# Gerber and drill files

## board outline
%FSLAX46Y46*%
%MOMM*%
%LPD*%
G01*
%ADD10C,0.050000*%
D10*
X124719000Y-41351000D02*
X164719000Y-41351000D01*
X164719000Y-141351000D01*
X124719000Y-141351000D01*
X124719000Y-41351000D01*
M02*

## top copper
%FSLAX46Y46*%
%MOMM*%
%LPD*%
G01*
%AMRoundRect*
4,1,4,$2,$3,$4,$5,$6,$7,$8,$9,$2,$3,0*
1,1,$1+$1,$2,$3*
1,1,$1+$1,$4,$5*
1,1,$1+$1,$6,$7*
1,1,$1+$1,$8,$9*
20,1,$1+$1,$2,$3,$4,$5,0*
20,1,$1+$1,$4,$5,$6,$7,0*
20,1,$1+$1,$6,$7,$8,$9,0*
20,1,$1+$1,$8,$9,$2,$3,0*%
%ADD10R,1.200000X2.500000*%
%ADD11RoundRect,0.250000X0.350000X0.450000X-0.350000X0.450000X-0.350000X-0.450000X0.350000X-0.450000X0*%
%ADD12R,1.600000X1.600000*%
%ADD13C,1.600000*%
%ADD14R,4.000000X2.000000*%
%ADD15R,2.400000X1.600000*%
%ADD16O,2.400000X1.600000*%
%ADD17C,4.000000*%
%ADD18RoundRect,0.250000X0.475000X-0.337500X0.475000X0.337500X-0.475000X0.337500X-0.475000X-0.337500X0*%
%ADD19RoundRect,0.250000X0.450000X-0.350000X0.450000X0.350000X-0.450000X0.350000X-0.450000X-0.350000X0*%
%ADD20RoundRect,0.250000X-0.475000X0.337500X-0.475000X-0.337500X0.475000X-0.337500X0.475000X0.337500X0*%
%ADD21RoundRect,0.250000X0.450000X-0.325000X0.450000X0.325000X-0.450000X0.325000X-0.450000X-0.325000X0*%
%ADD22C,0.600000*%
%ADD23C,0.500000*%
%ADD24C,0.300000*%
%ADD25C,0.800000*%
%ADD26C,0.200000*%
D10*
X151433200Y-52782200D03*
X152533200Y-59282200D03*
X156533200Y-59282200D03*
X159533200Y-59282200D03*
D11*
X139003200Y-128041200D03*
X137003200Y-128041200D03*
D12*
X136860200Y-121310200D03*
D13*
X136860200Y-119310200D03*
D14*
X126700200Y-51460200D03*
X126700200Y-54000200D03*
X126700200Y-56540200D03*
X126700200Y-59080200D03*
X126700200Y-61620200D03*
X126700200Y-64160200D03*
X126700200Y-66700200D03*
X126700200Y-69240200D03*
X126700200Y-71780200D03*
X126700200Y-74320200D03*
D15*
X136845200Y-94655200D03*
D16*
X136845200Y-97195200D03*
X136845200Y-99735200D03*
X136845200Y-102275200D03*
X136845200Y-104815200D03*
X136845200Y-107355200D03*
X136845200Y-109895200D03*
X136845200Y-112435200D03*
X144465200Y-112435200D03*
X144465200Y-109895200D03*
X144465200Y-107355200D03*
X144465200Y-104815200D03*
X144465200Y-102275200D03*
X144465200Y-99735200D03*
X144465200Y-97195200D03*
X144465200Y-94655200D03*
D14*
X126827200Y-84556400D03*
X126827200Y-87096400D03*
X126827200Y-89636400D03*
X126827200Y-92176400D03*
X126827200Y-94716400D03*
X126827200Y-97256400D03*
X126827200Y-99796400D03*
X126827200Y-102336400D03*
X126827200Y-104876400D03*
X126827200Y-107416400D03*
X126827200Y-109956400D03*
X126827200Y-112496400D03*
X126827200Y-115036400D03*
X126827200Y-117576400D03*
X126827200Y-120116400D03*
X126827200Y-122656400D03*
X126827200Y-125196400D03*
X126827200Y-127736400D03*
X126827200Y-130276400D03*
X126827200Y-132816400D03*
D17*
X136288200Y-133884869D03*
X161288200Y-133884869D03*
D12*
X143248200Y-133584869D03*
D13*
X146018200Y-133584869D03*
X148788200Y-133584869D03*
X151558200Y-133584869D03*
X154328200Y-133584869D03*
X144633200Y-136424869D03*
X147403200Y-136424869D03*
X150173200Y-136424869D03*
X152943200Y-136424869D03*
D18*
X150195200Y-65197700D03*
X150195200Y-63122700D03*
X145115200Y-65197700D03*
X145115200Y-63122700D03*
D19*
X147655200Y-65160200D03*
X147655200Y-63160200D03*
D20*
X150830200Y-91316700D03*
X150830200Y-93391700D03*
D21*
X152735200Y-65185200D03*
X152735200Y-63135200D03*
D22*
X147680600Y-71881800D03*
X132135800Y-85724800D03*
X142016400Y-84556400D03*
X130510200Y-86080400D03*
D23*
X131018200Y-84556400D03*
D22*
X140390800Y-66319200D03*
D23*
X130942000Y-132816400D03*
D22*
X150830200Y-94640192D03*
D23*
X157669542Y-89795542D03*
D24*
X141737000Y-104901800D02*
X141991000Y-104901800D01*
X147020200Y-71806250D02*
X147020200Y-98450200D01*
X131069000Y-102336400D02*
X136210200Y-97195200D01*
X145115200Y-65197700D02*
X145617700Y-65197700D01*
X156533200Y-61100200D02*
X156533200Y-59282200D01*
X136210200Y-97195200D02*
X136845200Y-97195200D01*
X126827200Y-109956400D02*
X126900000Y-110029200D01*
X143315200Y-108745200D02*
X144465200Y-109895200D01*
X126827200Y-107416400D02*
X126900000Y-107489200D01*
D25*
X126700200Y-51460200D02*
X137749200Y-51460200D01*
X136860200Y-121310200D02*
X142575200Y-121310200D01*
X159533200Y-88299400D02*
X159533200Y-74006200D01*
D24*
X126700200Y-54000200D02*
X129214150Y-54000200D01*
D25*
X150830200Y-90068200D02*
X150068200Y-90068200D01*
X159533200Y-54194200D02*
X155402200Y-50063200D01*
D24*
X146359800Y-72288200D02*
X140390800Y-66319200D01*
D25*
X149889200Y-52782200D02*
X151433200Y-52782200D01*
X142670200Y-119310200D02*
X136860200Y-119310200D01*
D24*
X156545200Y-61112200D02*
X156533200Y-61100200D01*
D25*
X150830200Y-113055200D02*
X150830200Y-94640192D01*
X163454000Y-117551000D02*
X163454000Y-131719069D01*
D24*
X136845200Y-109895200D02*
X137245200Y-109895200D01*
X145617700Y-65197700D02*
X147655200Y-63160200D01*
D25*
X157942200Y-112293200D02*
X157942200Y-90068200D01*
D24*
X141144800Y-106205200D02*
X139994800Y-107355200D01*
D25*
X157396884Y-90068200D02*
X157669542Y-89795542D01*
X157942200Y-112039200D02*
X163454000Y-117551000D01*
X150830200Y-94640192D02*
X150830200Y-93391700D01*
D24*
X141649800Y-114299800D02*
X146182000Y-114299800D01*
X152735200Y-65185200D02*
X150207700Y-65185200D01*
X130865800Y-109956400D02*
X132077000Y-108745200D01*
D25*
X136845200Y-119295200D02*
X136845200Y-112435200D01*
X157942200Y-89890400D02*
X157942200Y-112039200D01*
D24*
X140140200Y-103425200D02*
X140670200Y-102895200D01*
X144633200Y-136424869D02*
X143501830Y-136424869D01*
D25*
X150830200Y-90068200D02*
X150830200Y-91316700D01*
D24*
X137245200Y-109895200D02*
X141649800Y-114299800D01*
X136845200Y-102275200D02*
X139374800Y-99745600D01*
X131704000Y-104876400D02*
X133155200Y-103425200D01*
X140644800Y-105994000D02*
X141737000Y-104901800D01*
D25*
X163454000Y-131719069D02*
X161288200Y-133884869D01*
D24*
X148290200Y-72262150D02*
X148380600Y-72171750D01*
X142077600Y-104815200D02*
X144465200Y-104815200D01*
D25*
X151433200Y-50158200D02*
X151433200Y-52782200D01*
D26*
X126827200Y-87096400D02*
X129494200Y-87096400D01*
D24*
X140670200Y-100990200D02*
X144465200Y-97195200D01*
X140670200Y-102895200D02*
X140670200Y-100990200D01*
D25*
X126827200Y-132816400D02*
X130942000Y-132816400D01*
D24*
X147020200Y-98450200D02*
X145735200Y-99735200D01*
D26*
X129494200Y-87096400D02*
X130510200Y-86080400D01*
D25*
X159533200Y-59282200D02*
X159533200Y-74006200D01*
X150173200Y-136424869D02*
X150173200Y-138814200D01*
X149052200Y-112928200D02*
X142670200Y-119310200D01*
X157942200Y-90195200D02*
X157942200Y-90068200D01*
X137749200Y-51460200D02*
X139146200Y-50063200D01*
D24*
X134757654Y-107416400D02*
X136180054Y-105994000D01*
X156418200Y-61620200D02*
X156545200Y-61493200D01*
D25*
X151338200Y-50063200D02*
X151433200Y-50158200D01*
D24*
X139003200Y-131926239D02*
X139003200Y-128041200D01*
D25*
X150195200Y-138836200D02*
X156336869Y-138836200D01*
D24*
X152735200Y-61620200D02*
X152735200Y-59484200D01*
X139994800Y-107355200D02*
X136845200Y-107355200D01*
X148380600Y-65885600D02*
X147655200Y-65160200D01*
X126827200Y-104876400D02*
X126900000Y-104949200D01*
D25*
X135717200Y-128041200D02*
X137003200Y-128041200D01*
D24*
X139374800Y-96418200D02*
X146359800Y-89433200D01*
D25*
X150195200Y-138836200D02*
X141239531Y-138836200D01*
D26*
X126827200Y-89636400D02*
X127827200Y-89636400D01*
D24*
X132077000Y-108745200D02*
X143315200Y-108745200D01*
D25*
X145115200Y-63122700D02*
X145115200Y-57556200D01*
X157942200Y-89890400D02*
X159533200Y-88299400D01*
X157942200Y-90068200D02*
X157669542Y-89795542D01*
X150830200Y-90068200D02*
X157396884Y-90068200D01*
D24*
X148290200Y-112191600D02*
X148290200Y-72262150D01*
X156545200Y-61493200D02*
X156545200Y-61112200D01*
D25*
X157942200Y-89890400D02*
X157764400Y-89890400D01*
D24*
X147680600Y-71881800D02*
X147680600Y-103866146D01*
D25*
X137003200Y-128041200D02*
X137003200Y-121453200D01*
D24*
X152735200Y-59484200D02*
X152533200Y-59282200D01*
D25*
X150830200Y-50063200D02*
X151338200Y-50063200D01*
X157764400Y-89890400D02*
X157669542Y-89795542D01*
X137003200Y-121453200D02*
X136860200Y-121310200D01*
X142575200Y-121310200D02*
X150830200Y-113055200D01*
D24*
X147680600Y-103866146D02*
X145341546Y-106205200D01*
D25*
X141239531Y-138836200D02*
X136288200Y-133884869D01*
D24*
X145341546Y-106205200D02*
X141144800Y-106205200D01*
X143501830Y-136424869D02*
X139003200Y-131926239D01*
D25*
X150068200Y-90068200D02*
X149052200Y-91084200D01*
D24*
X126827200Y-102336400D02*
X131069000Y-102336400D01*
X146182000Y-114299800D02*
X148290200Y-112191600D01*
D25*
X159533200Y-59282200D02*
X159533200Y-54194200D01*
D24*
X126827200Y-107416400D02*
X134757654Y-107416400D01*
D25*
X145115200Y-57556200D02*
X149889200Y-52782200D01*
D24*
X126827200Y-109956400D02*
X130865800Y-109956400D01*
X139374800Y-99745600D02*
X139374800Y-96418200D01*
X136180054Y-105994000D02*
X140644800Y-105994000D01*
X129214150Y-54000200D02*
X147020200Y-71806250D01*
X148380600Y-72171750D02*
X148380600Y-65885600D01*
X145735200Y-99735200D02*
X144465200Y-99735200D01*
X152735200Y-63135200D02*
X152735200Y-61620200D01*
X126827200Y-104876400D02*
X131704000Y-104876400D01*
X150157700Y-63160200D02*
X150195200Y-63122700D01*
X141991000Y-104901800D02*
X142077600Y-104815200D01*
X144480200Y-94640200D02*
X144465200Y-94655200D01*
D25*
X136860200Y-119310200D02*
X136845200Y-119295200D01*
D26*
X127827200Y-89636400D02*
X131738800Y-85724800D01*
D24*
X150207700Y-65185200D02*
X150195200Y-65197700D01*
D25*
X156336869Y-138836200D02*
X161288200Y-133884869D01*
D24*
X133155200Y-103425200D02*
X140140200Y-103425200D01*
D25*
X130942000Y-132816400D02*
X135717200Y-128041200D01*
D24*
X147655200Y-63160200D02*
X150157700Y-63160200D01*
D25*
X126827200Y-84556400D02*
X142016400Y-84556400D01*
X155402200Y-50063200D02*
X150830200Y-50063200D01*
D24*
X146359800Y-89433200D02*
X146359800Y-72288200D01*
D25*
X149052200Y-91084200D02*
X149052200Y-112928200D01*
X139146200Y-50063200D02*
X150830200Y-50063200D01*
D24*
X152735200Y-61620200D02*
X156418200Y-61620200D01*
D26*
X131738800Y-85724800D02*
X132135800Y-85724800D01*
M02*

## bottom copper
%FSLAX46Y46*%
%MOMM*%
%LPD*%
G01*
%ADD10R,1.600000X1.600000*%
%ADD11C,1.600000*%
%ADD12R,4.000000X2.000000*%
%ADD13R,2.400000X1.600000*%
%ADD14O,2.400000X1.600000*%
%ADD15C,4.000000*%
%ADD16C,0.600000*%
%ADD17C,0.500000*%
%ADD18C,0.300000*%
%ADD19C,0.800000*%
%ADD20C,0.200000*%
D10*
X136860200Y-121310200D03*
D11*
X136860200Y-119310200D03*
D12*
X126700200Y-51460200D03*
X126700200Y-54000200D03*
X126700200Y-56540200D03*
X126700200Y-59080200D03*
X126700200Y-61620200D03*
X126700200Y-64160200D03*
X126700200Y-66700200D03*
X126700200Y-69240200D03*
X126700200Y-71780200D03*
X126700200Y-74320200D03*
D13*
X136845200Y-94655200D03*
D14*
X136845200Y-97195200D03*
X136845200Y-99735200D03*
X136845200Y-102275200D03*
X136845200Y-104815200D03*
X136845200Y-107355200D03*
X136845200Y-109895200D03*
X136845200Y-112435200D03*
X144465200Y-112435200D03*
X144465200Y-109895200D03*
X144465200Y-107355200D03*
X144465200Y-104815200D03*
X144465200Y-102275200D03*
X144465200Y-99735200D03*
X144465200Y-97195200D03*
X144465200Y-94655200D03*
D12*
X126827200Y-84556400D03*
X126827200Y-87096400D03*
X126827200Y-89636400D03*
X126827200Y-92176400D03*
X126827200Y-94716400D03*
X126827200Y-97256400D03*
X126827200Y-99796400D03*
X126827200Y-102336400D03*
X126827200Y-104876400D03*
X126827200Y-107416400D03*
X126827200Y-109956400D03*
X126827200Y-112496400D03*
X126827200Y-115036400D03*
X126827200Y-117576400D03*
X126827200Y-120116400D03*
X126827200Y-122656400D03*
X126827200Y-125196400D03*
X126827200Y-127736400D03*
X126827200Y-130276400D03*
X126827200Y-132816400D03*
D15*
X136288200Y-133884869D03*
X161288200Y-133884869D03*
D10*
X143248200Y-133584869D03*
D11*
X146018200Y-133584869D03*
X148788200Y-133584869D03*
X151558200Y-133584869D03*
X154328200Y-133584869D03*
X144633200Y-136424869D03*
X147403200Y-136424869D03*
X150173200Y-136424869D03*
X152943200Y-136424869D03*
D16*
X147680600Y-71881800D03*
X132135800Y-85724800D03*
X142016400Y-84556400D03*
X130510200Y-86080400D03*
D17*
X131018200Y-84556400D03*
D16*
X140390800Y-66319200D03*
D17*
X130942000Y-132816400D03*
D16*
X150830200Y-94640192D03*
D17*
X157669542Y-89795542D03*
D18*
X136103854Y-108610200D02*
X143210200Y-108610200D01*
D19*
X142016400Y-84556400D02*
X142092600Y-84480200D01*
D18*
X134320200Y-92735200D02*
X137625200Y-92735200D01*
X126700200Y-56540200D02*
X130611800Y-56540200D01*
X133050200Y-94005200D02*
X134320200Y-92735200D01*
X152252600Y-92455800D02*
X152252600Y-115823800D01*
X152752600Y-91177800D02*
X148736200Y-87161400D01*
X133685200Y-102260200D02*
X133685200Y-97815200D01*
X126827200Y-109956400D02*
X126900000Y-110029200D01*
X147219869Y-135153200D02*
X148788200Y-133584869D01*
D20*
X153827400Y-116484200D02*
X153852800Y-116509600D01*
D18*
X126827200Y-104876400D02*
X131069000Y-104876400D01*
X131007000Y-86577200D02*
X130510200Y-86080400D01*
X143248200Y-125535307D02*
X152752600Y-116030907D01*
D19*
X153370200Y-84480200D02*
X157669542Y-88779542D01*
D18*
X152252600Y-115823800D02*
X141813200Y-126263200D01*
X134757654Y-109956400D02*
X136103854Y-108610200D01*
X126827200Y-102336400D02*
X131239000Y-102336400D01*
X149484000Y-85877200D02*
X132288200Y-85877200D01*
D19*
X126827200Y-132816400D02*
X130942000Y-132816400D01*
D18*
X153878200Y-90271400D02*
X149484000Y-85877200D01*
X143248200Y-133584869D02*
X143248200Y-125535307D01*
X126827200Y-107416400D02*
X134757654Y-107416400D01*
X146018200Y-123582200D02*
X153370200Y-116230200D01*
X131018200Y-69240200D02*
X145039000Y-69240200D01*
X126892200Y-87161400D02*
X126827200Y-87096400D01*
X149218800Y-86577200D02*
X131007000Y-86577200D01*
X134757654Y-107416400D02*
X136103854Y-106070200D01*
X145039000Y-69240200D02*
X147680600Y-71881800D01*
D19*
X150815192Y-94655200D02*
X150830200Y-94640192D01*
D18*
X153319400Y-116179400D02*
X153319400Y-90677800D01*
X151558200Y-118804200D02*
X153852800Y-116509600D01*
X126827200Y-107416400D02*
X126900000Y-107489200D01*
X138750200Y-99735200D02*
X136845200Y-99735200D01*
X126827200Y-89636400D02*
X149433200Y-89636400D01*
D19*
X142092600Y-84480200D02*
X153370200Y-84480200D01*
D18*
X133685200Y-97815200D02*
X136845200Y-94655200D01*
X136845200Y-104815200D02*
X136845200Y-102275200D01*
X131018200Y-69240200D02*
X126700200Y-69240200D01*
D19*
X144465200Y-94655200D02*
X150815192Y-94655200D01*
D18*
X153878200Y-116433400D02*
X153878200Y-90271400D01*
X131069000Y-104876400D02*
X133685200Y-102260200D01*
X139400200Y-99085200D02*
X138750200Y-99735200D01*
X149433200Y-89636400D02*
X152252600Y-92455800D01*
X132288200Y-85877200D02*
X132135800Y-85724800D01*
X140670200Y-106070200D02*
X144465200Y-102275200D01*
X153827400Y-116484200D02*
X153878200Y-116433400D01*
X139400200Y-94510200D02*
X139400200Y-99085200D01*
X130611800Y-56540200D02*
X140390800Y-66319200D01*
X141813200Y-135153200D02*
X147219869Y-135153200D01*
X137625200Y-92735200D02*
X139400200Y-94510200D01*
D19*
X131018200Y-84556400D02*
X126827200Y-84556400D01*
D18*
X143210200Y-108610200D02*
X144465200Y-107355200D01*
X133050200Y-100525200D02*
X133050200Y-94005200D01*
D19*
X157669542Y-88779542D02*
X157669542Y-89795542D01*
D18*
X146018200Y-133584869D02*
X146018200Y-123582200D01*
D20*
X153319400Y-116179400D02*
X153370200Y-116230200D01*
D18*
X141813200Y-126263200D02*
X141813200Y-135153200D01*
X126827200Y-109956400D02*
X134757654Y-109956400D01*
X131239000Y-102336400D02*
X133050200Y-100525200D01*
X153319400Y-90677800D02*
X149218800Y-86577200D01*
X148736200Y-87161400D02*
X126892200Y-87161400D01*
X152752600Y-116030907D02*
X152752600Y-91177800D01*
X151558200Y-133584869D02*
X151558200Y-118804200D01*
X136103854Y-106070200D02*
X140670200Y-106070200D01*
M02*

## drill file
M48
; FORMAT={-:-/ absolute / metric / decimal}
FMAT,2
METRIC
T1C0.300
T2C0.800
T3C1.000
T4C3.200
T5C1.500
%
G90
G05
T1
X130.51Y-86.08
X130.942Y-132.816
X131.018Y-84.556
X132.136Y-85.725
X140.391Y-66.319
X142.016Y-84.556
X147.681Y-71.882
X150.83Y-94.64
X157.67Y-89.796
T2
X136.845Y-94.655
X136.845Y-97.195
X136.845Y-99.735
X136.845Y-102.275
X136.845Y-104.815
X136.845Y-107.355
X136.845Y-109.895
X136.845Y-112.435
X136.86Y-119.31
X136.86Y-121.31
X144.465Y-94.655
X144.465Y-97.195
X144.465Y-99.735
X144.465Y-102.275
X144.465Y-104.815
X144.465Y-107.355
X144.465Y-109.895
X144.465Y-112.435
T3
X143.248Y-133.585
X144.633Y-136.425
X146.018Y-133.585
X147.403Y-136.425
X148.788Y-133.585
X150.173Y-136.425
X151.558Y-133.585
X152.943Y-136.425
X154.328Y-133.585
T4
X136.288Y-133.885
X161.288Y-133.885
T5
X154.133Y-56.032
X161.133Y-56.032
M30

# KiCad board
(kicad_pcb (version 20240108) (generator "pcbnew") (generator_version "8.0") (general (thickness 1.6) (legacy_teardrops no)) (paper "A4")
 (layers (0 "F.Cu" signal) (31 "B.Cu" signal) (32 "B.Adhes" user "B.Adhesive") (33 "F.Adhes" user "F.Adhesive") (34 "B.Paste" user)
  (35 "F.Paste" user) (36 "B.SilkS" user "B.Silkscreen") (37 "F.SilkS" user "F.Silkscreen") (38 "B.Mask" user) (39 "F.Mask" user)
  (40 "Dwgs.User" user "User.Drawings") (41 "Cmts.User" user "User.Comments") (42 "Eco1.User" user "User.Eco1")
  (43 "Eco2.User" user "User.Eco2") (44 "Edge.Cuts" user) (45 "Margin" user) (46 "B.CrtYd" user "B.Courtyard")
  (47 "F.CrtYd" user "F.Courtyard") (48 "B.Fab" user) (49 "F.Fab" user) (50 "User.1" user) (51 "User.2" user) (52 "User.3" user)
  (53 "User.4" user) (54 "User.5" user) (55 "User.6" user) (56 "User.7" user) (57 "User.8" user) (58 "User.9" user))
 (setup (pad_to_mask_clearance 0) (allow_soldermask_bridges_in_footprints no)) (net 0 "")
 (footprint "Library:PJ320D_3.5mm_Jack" (layer "F.Cu") (at 156.3582 56.0322 180)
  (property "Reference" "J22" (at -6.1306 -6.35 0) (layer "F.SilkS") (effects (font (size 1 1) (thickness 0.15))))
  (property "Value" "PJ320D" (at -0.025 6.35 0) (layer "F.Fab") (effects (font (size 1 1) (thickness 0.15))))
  (pad "" np_thru_hole circle (at -4.775 0 180) (size 1.5 1.5) (drill 1.5) (layers "*.Cu" "*.Mask"))
  (pad "" np_thru_hole circle (at 2.225 0 180) (size 1.5 1.5) (drill 1.5) (layers "*.Cu" "*.Mask"))
  (pad "1" smd rect (at 4.925 3.25 180) (size 1.2 2.5) (layers "F.Cu" "F.Paste" "F.Mask"))
  (pad "2" smd rect (at 3.825 -3.25 180) (size 1.2 2.5) (layers "F.Cu" "F.Paste" "F.Mask"))
  (pad "3" smd rect (at -0.175 -3.25 180) (size 1.2 2.5) (layers "F.Cu" "F.Paste" "F.Mask"))
  (pad "4" smd rect (at -3.175 -3.25 180) (size 1.2 2.5) (layers "F.Cu" "F.Paste" "F.Mask")))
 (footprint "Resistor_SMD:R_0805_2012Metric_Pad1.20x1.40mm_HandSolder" (layer "F.Cu") (at 138.0032 128.0412 180)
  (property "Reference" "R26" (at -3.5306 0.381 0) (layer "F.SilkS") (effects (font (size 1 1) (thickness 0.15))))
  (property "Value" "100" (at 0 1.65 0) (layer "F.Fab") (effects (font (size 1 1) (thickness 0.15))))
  (pad "1" smd roundrect (at -1 0 180) (size 1.2 1.4) (layers "F.Cu" "F.Paste" "F.Mask") (roundrect_rratio 0.208333))
  (pad "2" smd roundrect (at 1 0 180) (size 1.2 1.4) (layers "F.Cu" "F.Paste" "F.Mask") (roundrect_rratio 0.208333)))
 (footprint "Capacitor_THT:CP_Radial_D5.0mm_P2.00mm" (layer "F.Cu") (at 136.8602 121.3102 90)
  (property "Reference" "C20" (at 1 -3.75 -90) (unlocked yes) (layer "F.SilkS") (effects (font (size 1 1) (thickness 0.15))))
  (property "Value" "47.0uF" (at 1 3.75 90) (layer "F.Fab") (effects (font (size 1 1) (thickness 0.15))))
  (pad "1" thru_hole rect (at 0 0 90) (size 1.6 1.6) (drill 0.8) (layers "*.Cu" "*.Mask") (remove_unused_layers no))
  (pad "2" thru_hole circle (at 2 0 90) (size 1.6 1.6) (drill 0.8) (layers "*.Cu" "*.Mask") (remove_unused_layers no)))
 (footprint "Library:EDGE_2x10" (layer "F.Cu") (at 126.7002 51.4602 -90)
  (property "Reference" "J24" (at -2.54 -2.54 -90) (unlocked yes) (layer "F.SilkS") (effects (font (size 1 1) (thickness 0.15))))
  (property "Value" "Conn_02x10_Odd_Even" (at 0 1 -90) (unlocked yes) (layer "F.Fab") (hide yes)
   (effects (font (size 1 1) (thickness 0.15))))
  (pad "1" connect rect (at 0 0 270) (size 2 4) (layers "B.Cu" "B.Mask") (thermal_bridge_angle 45))
  (pad "2" connect rect (at 0 0 270) (size 2 4) (layers "F.Cu" "F.Mask") (thermal_bridge_angle 45))
  (pad "3" connect rect (at 2.54 0 270) (size 2 4) (layers "B.Cu" "B.Mask") (thermal_bridge_angle 45))
  (pad "4" connect rect (at 2.54 0 270) (size 2 4) (layers "F.Cu" "F.Mask") (thermal_bridge_angle 45))
  (pad "5" connect rect (at 5.08 0 270) (size 2 4) (layers "B.Cu" "B.Mask") (thermal_bridge_angle 45))
  (pad "6" connect rect (at 5.08 0 270) (size 2 4) (layers "F.Cu" "F.Mask") (thermal_bridge_angle 45))
  (pad "7" connect rect (at 7.62 0 270) (size 2 4) (layers "B.Cu" "B.Mask") (thermal_bridge_angle 45))
  (pad "8" connect rect (at 7.62 0 270) (size 2 4) (layers "F.Cu" "F.Mask") (thermal_bridge_angle 45))
  (pad "9" connect rect (at 10.16 0 270) (size 2 4) (layers "B.Cu" "B.Mask") (thermal_bridge_angle 45))
  (pad "10" connect rect (at 10.16 0 270) (size 2 4) (layers "F.Cu" "F.Mask") (thermal_bridge_angle 45))
  (pad "11" connect rect (at 12.7 0 270) (size 2 4) (layers "B.Cu" "B.Mask") (thermal_bridge_angle 45))
  (pad "12" connect rect (at 12.7 0 270) (size 2 4) (layers "F.Cu" "F.Mask") (thermal_bridge_angle 45))
  (pad "13" connect rect (at 15.24 0 270) (size 2 4) (layers "B.Cu" "B.Mask") (thermal_bridge_angle 45))
  (pad "14" connect rect (at 15.24 0 270) (size 2 4) (layers "F.Cu" "F.Mask") (thermal_bridge_angle 45))
  (pad "15" connect rect (at 17.78 0 270) (size 2 4) (layers "B.Cu" "B.Mask") (thermal_bridge_angle 45))
  (pad "16" connect rect (at 17.78 0 270) (size 2 4) (layers "F.Cu" "F.Mask") (thermal_bridge_angle 45))
  (pad "17" connect rect (at 20.32 0 270) (size 2 4) (layers "B.Cu" "B.Mask") (thermal_bridge_angle 45))
  (pad "18" connect rect (at 20.32 0 270) (size 2 4) (layers "F.Cu" "F.Mask") (thermal_bridge_angle 45))
  (pad "19" connect rect (at 22.86 0 270) (size 2 4) (layers "B.Cu" "B.Mask") (thermal_bridge_angle 45))
  (pad "20" connect rect (at 22.86 0 270) (size 2 4) (layers "F.Cu" "F.Mask") (thermal_bridge_angle 45)))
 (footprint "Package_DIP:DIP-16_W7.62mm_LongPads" (layer "F.Cu") (at 136.8452 94.6552)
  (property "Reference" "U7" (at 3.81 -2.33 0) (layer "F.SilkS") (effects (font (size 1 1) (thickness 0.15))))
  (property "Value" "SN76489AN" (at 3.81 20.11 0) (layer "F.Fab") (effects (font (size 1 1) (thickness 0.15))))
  (pad "1" thru_hole rect (at 0 0) (size 2.4 1.6) (drill 0.8) (layers "*.Cu" "*.Mask") (remove_unused_layers no))
  (pad "2" thru_hole oval (at 0 2.54) (size 2.4 1.6) (drill 0.8) (layers "*.Cu" "*.Mask") (remove_unused_layers no))
  (pad "3" thru_hole oval (at 0 5.08) (size 2.4 1.6) (drill 0.8) (layers "*.Cu" "*.Mask") (remove_unused_layers no))
  (pad "4" thru_hole oval (at 0 7.62) (size 2.4 1.6) (drill 0.8) (layers "*.Cu" "*.Mask") (remove_unused_layers no))
  (pad "5" thru_hole oval (at 0 10.16) (size 2.4 1.6) (drill 0.8) (layers "*.Cu" "*.Mask") (remove_unused_layers no))
  (pad "6" thru_hole oval (at 0 12.7) (size 2.4 1.6) (drill 0.8) (layers "*.Cu" "*.Mask") (remove_unused_layers no))
  (pad "7" thru_hole oval (at 0 15.24) (size 2.4 1.6) (drill 0.8) (layers "*.Cu" "*.Mask") (remove_unused_layers no))
  (pad "8" thru_hole oval (at 0 17.78) (size 2.4 1.6) (drill 0.8) (layers "*.Cu" "*.Mask") (remove_unused_layers no))
  (pad "9" thru_hole oval (at 7.62 17.78) (size 2.4 1.6) (drill 0.8) (layers "*.Cu" "*.Mask") (remove_unused_layers no))
  (pad "10" thru_hole oval (at 7.62 15.24) (size 2.4 1.6) (drill 0.8) (layers "*.Cu" "*.Mask") (remove_unused_layers no))
  (pad "11" thru_hole oval (at 7.62 12.7) (size 2.4 1.6) (drill 0.8) (layers "*.Cu" "*.Mask") (remove_unused_layers no))
  (pad "12" thru_hole oval (at 7.62 10.16) (size 2.4 1.6) (drill 0.8) (layers "*.Cu" "*.Mask") (remove_unused_layers no))
  (pad "13" thru_hole oval (at 7.62 7.62) (size 2.4 1.6) (drill 0.8) (layers "*.Cu" "*.Mask") (remove_unused_layers no))
  (pad "14" thru_hole oval (at 7.62 5.08) (size 2.4 1.6) (drill 0.8) (layers "*.Cu" "*.Mask") (remove_unused_layers no))
  (pad "15" thru_hole oval (at 7.62 2.54) (size 2.4 1.6) (drill 0.8) (layers "*.Cu" "*.Mask") (remove_unused_layers no))
  (pad "16" thru_hole oval (at 7.62 0) (size 2.4 1.6) (drill 0.8) (layers "*.Cu" "*.Mask") (remove_unused_layers no)))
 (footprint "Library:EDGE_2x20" (layer "F.Cu") (at 126.8272 84.5564 -90)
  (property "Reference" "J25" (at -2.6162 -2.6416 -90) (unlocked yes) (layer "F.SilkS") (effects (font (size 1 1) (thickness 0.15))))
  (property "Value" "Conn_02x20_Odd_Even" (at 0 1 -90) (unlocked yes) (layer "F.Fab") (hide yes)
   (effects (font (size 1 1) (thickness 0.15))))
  (pad "1" connect rect (at 0 0 270) (size 2 4) (layers "B.Cu" "B.Mask") (thermal_bridge_angle 45))
  (pad "2" connect rect (at 0 0 270) (size 2 4) (layers "F.Cu" "F.Mask") (thermal_bridge_angle 45))
  (pad "3" connect rect (at 2.54 0 270) (size 2 4) (layers "B.Cu" "B.Mask") (thermal_bridge_angle 45))
  (pad "4" connect rect (at 2.54 0 270) (size 2 4) (layers "F.Cu" "F.Mask") (thermal_bridge_angle 45))
  (pad "5" connect rect (at 5.08 0 270) (size 2 4) (layers "B.Cu" "B.Mask") (thermal_bridge_angle 45))
  (pad "6" connect rect (at 5.08 0 270) (size 2 4) (layers "F.Cu" "F.Mask") (thermal_bridge_angle 45))
  (pad "7" connect rect (at 7.62 0 270) (size 2 4) (layers "B.Cu" "B.Mask") (thermal_bridge_angle 45))
  (pad "8" connect rect (at 7.62 0 270) (size 2 4) (layers "F.Cu" "F.Mask") (thermal_bridge_angle 45))
  (pad "9" connect rect (at 10.16 0 270) (size 2 4) (layers "B.Cu" "B.Mask") (thermal_bridge_angle 45))
  (pad "10" connect rect (at 10.16 0 270) (size 2 4) (layers "F.Cu" "F.Mask") (thermal_bridge_angle 45))
  (pad "11" connect rect (at 12.7 0 270) (size 2 4) (layers "B.Cu" "B.Mask") (thermal_bridge_angle 45))
  (pad "12" connect rect (at 12.7 0 270) (size 2 4) (layers "F.Cu" "F.Mask") (thermal_bridge_angle 45))
  (pad "13" connect rect (at 15.24 0 270) (size 2 4) (layers "B.Cu" "B.Mask") (thermal_bridge_angle 45))
  (pad "14" connect rect (at 15.24 0 270) (size 2 4) (layers "F.Cu" "F.Mask") (thermal_bridge_angle 45))
  (pad "15" connect rect (at 17.78 0 270) (size 2 4) (layers "B.Cu" "B.Mask") (thermal_bridge_angle 45))
  (pad "16" connect rect (at 17.78 0 270) (size 2 4) (layers "F.Cu" "F.Mask") (thermal_bridge_angle 45))
  (pad "17" connect rect (at 20.32 0 270) (size 2 4) (layers "B.Cu" "B.Mask") (thermal_bridge_angle 45))
  (pad "18" connect rect (at 20.32 0 270) (size 2 4) (layers "F.Cu" "F.Mask") (thermal_bridge_angle 45))
  (pad "19" connect rect (at 22.86 0 270) (size 2 4) (layers "B.Cu" "B.Mask") (thermal_bridge_angle 45))
  (pad "20" connect rect (at 22.86 0 270) (size 2 4) (layers "F.Cu" "F.Mask") (thermal_bridge_angle 45))
  (pad "21" connect rect (at 25.4 0 270) (size 2 4) (layers "B.Cu" "B.Mask") (thermal_bridge_angle 45))
  (pad "22" connect rect (at 25.4 0 270) (size 2 4) (layers "F.Cu" "F.Mask") (thermal_bridge_angle 45))
  (pad "23" connect rect (at 27.94 0 270) (size 2 4) (layers "B.Cu" "B.Mask") (thermal_bridge_angle 45))
  (pad "24" connect rect (at 27.94 0 270) (size 2 4) (layers "F.Cu" "F.Mask") (thermal_bridge_angle 45))
  (pad "25" connect rect (at 30.48 0 270) (size 2 4) (layers "B.Cu" "B.Mask") (thermal_bridge_angle 45))
  (pad "26" connect rect (at 30.48 0 270) (size 2 4) (layers "F.Cu" "F.Mask") (thermal_bridge_angle 45))
  (pad "27" connect rect (at 33.02 0 270) (size 2 4) (layers "B.Cu" "B.Mask") (thermal_bridge_angle 45))
  (pad "28" connect rect (at 33.02 0 270) (size 2 4) (layers "F.Cu" "F.Mask") (thermal_bridge_angle 45))
  (pad "29" connect rect (at 35.56 0 270) (size 2 4) (layers "B.Cu" "B.Mask") (thermal_bridge_angle 45))
  (pad "30" connect rect (at 35.56 0 270) (size 2 4) (layers "F.Cu" "F.Mask") (thermal_bridge_angle 45))
  (pad "31" connect rect (at 38.1 0 270) (size 2 4) (layers "B.Cu" "B.Mask") (thermal_bridge_angle 45))
  (pad "32" connect rect (at 38.1 0 270) (size 2 4) (layers "F.Cu" "F.Mask") (thermal_bridge_angle 45))
  (pad "33" connect rect (at 40.64 0 270) (size 2 4) (layers "B.Cu" "B.Mask") (thermal_bridge_angle 45))
  (pad "34" connect rect (at 40.64 0 270) (size 2 4) (layers "F.Cu" "F.Mask") (thermal_bridge_angle 45))
  (pad "35" connect rect (at 43.18 0 270) (size 2 4) (layers "B.Cu" "B.Mask") (thermal_bridge_angle 45))
  (pad "36" connect rect (at 43.18 0 270) (size 2 4) (layers "F.Cu" "F.Mask") (thermal_bridge_angle 45))
  (pad "37" connect rect (at 45.72 0 270) (size 2 4) (layers "B.Cu" "B.Mask") (thermal_bridge_angle 45))
  (pad "38" connect rect (at 45.72 0 270) (size 2 4) (layers "F.Cu" "F.Mask") (thermal_bridge_angle 45))
  (pad "39" connect rect (at 48.26 0 270) (size 2 4) (layers "B.Cu" "B.Mask") (thermal_bridge_angle 45))
  (pad "40" connect rect (at 48.26 0 270) (size 2 4) (layers "F.Cu" "F.Mask") (thermal_bridge_angle 45)))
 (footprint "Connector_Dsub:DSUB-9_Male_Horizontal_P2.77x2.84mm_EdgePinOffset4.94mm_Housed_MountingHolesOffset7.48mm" (layer "F.Cu")
  (at 143.2482 133.584869)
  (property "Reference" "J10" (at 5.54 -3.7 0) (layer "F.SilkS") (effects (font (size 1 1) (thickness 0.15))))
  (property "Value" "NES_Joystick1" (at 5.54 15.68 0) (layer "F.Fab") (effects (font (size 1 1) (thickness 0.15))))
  (pad "0" thru_hole circle (at -6.96 0.3) (size 4 4) (drill 3.2) (layers "*.Cu" "*.Mask") (remove_unused_layers no))
  (pad "0" thru_hole circle (at 18.04 0.3) (size 4 4) (drill 3.2) (layers "*.Cu" "*.Mask") (remove_unused_layers no))
  (pad "1" thru_hole rect (at 0 0) (size 1.6 1.6) (drill 1) (layers "*.Cu" "*.Mask") (remove_unused_layers no))
  (pad "2" thru_hole circle (at 2.77 0) (size 1.6 1.6) (drill 1) (layers "*.Cu" "*.Mask") (remove_unused_layers no))
  (pad "3" thru_hole circle (at 5.54 0) (size 1.6 1.6) (drill 1) (layers "*.Cu" "*.Mask") (remove_unused_layers no))
  (pad "4" thru_hole circle (at 8.31 0) (size 1.6 1.6) (drill 1) (layers "*.Cu" "*.Mask") (remove_unused_layers no))
  (pad "5" thru_hole circle (at 11.08 0) (size 1.6 1.6) (drill 1) (layers "*.Cu" "*.Mask") (remove_unused_layers no))
  (pad "6" thru_hole circle (at 1.385 2.84) (size 1.6 1.6) (drill 1) (layers "*.Cu" "*.Mask") (remove_unused_layers no))
  (pad "7" thru_hole circle (at 4.155 2.84) (size 1.6 1.6) (drill 1) (layers "*.Cu" "*.Mask") (remove_unused_layers no))
  (pad "8" thru_hole circle (at 6.925 2.84) (size 1.6 1.6) (drill 1) (layers "*.Cu" "*.Mask") (remove_unused_layers no))
  (pad "9" thru_hole circle (at 9.695 2.84) (size 1.6 1.6) (drill 1) (layers "*.Cu" "*.Mask") (remove_unused_layers no)))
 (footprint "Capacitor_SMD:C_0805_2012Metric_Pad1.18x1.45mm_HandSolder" (layer "F.Cu") (at 150.1952 64.1602 90)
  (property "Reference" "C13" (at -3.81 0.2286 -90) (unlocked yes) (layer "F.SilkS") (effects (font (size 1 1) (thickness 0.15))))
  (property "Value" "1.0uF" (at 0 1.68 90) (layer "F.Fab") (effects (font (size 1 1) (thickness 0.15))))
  (pad "1" smd roundrect (at -1.0375 0 90) (size 1.175 1.45) (layers "F.Cu" "F.Paste" "F.Mask") (roundrect_rratio 0.212766))
  (pad "2" smd roundrect (at 1.0375 0 90) (size 1.175 1.45) (layers "F.Cu" "F.Paste" "F.Mask") (roundrect_rratio 0.212766)))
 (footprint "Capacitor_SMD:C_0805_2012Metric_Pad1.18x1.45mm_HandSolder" (layer "F.Cu") (at 145.1152 64.1602 90)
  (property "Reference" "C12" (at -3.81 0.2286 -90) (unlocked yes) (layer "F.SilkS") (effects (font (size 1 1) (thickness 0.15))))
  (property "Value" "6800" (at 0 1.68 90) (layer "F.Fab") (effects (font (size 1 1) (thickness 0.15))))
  (pad "1" smd roundrect (at -1.0375 0 90) (size 1.175 1.45) (layers "F.Cu" "F.Paste" "F.Mask") (roundrect_rratio 0.212766))
  (pad "2" smd roundrect (at 1.0375 0 90) (size 1.175 1.45) (layers "F.Cu" "F.Paste" "F.Mask") (roundrect_rratio 0.212766)))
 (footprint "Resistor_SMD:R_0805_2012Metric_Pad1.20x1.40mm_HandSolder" (layer "F.Cu") (at 147.6552 64.1602 90)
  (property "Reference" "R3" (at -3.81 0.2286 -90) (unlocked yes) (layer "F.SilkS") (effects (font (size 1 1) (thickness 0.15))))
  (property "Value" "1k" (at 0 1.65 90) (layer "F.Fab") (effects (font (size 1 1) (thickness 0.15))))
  (pad "1" smd roundrect (at -1 0 90) (size 1.2 1.4) (layers "F.Cu" "F.Paste" "F.Mask") (roundrect_rratio 0.208333))
  (pad "2" smd roundrect (at 1 0 90) (size 1.2 1.4) (layers "F.Cu" "F.Paste" "F.Mask") (roundrect_rratio 0.208333)))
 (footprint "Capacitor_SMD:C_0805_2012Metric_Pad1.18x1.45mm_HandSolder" (layer "F.Cu") (at 150.8302 92.3542 -90)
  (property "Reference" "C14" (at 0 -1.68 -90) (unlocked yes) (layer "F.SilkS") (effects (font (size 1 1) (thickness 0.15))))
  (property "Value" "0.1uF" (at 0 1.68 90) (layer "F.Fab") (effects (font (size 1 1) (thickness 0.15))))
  (pad "1" smd roundrect (at -1.0375 0 270) (size 1.175 1.45) (layers "F.Cu" "F.Paste" "F.Mask") (roundrect_rratio 0.212766))
  (pad "2" smd roundrect (at 1.0375 0 270) (size 1.175 1.45) (layers "F.Cu" "F.Paste" "F.Mask") (roundrect_rratio 0.212766)))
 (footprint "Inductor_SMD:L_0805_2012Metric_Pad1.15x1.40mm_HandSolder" (layer "F.Cu") (at 152.7352 64.1602 90)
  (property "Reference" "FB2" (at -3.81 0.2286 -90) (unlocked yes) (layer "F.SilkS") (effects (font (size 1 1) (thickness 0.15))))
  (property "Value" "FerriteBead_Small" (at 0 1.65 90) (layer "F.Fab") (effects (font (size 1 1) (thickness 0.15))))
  (pad "1" smd roundrect (at -1.025 0 90) (size 1.15 1.4) (layers "F.Cu" "F.Paste" "F.Mask") (roundrect_rratio 0.217391))
  (pad "2" smd roundrect (at 1.025 0 90) (size 1.15 1.4) (layers "F.Cu" "F.Paste" "F.Mask") (roundrect_rratio 0.217391)))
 (gr_rect (start 124.719 41.351) (end 164.719 141.351) (stroke (width 0.05) (type default)) (fill none) (layer "Edge.Cuts"))
 (segment (start 141.737 104.9018) (end 141.991 104.9018) (width 0.3) (layer "F.Cu") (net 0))
 (segment (start 147.0202 71.80625) (end 147.0202 98.4502) (width 0.3) (layer "F.Cu") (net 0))
 (segment (start 131.069 102.3364) (end 136.2102 97.1952) (width 0.3) (layer "F.Cu") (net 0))
 (segment (start 145.1152 65.1977) (end 145.6177 65.1977) (width 0.3) (layer "F.Cu") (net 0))
 (segment (start 156.5332 61.1002) (end 156.5332 59.2822) (width 0.3) (layer "F.Cu") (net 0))
 (segment (start 136.2102 97.1952) (end 136.8452 97.1952) (width 0.3) (layer "F.Cu") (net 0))
 (segment (start 126.8272 109.9564) (end 126.9 110.0292) (width 0.3) (layer "F.Cu") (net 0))
 (segment (start 143.3152 108.7452) (end 144.4652 109.8952) (width 0.3) (layer "F.Cu") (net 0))
 (segment (start 126.8272 107.4164) (end 126.9 107.4892) (width 0.3) (layer "F.Cu") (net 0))
 (segment (start 126.7002 51.4602) (end 137.7492 51.4602) (width 0.8) (layer "F.Cu") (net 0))
 (segment (start 136.8602 121.3102) (end 142.5752 121.3102) (width 0.8) (layer "F.Cu") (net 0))
 (segment (start 159.5332 88.2994) (end 159.5332 74.0062) (width 0.8) (layer "F.Cu") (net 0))
 (segment (start 126.7002 54.0002) (end 129.21415 54.0002) (width 0.3) (layer "F.Cu") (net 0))
 (segment (start 150.8302 90.0682) (end 150.0682 90.0682) (width 0.8) (layer "F.Cu") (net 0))
 (segment (start 159.5332 54.1942) (end 155.4022 50.0632) (width 0.8) (layer "F.Cu") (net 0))
 (segment (start 146.3598 72.2882) (end 140.3908 66.3192) (width 0.3) (layer "F.Cu") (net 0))
 (segment (start 149.8892 52.7822) (end 151.4332 52.7822) (width 0.8) (layer "F.Cu") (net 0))
 (segment (start 142.6702 119.3102) (end 136.8602 119.3102) (width 0.8) (layer "F.Cu") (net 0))
 (segment (start 156.5452 61.1122) (end 156.5332 61.1002) (width 0.3) (layer "F.Cu") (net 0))
 (segment (start 150.8302 113.0552) (end 150.8302 94.640192) (width 0.8) (layer "F.Cu") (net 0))
 (segment (start 163.454 117.551) (end 163.454 131.719069) (width 0.8) (layer "F.Cu") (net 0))
 (segment (start 136.8452 109.8952) (end 137.2452 109.8952) (width 0.3) (layer "F.Cu") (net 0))
 (segment (start 145.6177 65.1977) (end 147.6552 63.1602) (width 0.3) (layer "F.Cu") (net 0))
 (segment (start 157.9422 112.2932) (end 157.9422 90.0682) (width 0.8) (layer "F.Cu") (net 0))
 (segment (start 141.1448 106.2052) (end 139.9948 107.3552) (width 0.3) (layer "F.Cu") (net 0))
 (segment (start 157.396884 90.0682) (end 157.669542 89.795542) (width 0.8) (layer "F.Cu") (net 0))
 (segment (start 157.9422 112.0392) (end 163.454 117.551) (width 0.8) (layer "F.Cu") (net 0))
 (segment (start 150.8302 94.640192) (end 150.8302 93.3917) (width 0.8) (layer "F.Cu") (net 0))
 (segment (start 141.6498 114.2998) (end 146.182 114.2998) (width 0.3) (layer "F.Cu") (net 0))
 (segment (start 152.7352 65.1852) (end 150.2077 65.1852) (width 0.3) (layer "F.Cu") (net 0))
 (segment (start 130.8658 109.9564) (end 132.077 108.7452) (width 0.3) (layer "F.Cu") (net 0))
 (segment (start 136.8452 119.2952) (end 136.8452 112.4352) (width 0.8) (layer "F.Cu") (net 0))
 (segment (start 157.9422 89.8904) (end 157.9422 112.0392) (width 0.8) (layer "F.Cu") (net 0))
 (segment (start 140.1402 103.4252) (end 140.6702 102.8952) (width 0.3) (layer "F.Cu") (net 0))
 (segment (start 144.6332 136.424869) (end 143.50183 136.424869) (width 0.3) (layer "F.Cu") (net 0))
 (segment (start 150.8302 90.0682) (end 150.8302 91.3167) (width 0.8) (layer "F.Cu") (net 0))
 (segment (start 137.2452 109.8952) (end 141.6498 114.2998) (width 0.3) (layer "F.Cu") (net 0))
 (segment (start 136.8452 102.2752) (end 139.3748 99.7456) (width 0.3) (layer "F.Cu") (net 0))
 (segment (start 131.704 104.8764) (end 133.1552 103.4252) (width 0.3) (layer "F.Cu") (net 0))
 (segment (start 140.6448 105.994) (end 141.737 104.9018) (width 0.3) (layer "F.Cu") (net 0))
 (segment (start 163.454 131.719069) (end 161.2882 133.884869) (width 0.8) (layer "F.Cu") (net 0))
 (segment (start 148.2902 72.26215) (end 148.3806 72.17175) (width 0.3) (layer "F.Cu") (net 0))
 (segment (start 142.0776 104.8152) (end 144.4652 104.8152) (width 0.3) (layer "F.Cu") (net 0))
 (segment (start 151.4332 50.1582) (end 151.4332 52.7822) (width 0.8) (layer "F.Cu") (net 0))
 (segment (start 126.8272 87.0964) (end 129.4942 87.0964) (width 0.2) (layer "F.Cu") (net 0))
 (segment (start 140.6702 100.9902) (end 144.4652 97.1952) (width 0.3) (layer "F.Cu") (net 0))
 (segment (start 140.6702 102.8952) (end 140.6702 100.9902) (width 0.3) (layer "F.Cu") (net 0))
 (segment (start 126.8272 132.8164) (end 130.942 132.8164) (width 0.8) (layer "F.Cu") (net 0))
 (segment (start 147.0202 98.4502) (end 145.7352 99.7352) (width 0.3) (layer "F.Cu") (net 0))
 (segment (start 129.4942 87.0964) (end 130.5102 86.0804) (width 0.2) (layer "F.Cu") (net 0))
 (segment (start 159.5332 59.2822) (end 159.5332 74.0062) (width 0.8) (layer "F.Cu") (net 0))
 (segment (start 150.1732 136.424869) (end 150.1732 138.8142) (width 0.8) (layer "F.Cu") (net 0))
 (segment (start 149.0522 112.9282) (end 142.6702 119.3102) (width 0.8) (layer "F.Cu") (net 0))
 (segment (start 157.9422 90.1952) (end 157.9422 90.0682) (width 0.8) (layer "F.Cu") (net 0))
 (segment (start 137.7492 51.4602) (end 139.1462 50.0632) (width 0.8) (layer "F.Cu") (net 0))
 (segment (start 134.757654 107.4164) (end 136.180054 105.994) (width 0.3) (layer "F.Cu") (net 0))
 (segment (start 156.4182 61.6202) (end 156.5452 61.4932) (width 0.3) (layer "F.Cu") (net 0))
 (segment (start 151.3382 50.0632) (end 151.4332 50.1582) (width 0.8) (layer "F.Cu") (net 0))
 (segment (start 139.0032 131.926239) (end 139.0032 128.0412) (width 0.3) (layer "F.Cu") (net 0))
 (segment (start 150.1952 138.8362) (end 156.336869 138.8362) (width 0.8) (layer "F.Cu") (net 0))
 (segment (start 152.7352 61.6202) (end 152.7352 59.4842) (width 0.3) (layer "F.Cu") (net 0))
 (segment (start 139.9948 107.3552) (end 136.8452 107.3552) (width 0.3) (layer "F.Cu") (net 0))
 (segment (start 148.3806 65.8856) (end 147.6552 65.1602) (width 0.3) (layer "F.Cu") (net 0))
 (segment (start 126.8272 104.8764) (end 126.9 104.9492) (width 0.3) (layer "F.Cu") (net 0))
 (segment (start 135.7172 128.0412) (end 137.0032 128.0412) (width 0.8) (layer "F.Cu") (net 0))
 (segment (start 139.3748 96.4182) (end 146.3598 89.4332) (width 0.3) (layer "F.Cu") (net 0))
 (segment (start 150.1952 138.8362) (end 141.239531 138.8362) (width 0.8) (layer "F.Cu") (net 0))
 (segment (start 126.8272 89.6364) (end 127.8272 89.6364) (width 0.2) (layer "F.Cu") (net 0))
 (segment (start 132.077 108.7452) (end 143.3152 108.7452) (width 0.3) (layer "F.Cu") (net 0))
 (segment (start 145.1152 63.1227) (end 145.1152 57.5562) (width 0.8) (layer "F.Cu") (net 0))
 (segment (start 157.9422 89.8904) (end 159.5332 88.2994) (width 0.8) (layer "F.Cu") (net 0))
 (segment (start 157.9422 90.0682) (end 157.669542 89.795542) (width 0.8) (layer "F.Cu") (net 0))
 (segment (start 150.8302 90.0682) (end 157.396884 90.0682) (width 0.8) (layer "F.Cu") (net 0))
 (segment (start 148.2902 112.1916) (end 148.2902 72.26215) (width 0.3) (layer "F.Cu") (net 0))
 (segment (start 156.5452 61.4932) (end 156.5452 61.1122) (width 0.3) (layer "F.Cu") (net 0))
 (segment (start 157.9422 89.8904) (end 157.7644 89.8904) (width 0.8) (layer "F.Cu") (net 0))
 (segment (start 147.6806 71.8818) (end 147.6806 103.866146) (width 0.3) (layer "F.Cu") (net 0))
 (segment (start 137.0032 128.0412) (end 137.0032 121.4532) (width 0.8) (layer "F.Cu") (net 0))
 (segment (start 152.7352 59.4842) (end 152.5332 59.2822) (width 0.3) (layer "F.Cu") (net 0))
 (segment (start 150.8302 50.0632) (end 151.3382 50.0632) (width 0.8) (layer "F.Cu") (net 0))
 (segment (start 157.7644 89.8904) (end 157.669542 89.795542) (width 0.8) (layer "F.Cu") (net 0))
 (segment (start 137.0032 121.4532) (end 136.8602 121.3102) (width 0.8) (layer "F.Cu") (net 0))
 (segment (start 142.5752 121.3102) (end 150.8302 113.0552) (width 0.8) (layer "F.Cu") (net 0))
 (segment (start 147.6806 103.866146) (end 145.341546 106.2052) (width 0.3) (layer "F.Cu") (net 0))
 (segment (start 141.239531 138.8362) (end 136.2882 133.884869) (width 0.8) (layer "F.Cu") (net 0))
 (segment (start 145.341546 106.2052) (end 141.1448 106.2052) (width 0.3) (layer "F.Cu") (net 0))
 (segment (start 143.50183 136.424869) (end 139.0032 131.926239) (width 0.3) (layer "F.Cu") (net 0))
 (segment (start 150.0682 90.0682) (end 149.0522 91.0842) (width 0.8) (layer "F.Cu") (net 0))
 (segment (start 126.8272 102.3364) (end 131.069 102.3364) (width 0.3) (layer "F.Cu") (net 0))
 (segment (start 146.182 114.2998) (end 148.2902 112.1916) (width 0.3) (layer "F.Cu") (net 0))
 (segment (start 159.5332 59.2822) (end 159.5332 54.1942) (width 0.8) (layer "F.Cu") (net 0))
 (segment (start 126.8272 107.4164) (end 134.757654 107.4164) (width 0.3) (layer "F.Cu") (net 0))
 (segment (start 145.1152 57.5562) (end 149.8892 52.7822) (width 0.8) (layer "F.Cu") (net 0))
 (segment (start 126.8272 109.9564) (end 130.8658 109.9564) (width 0.3) (layer "F.Cu") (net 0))
 (segment (start 139.3748 99.7456) (end 139.3748 96.4182) (width 0.3) (layer "F.Cu") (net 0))
 (segment (start 136.180054 105.994) (end 140.6448 105.994) (width 0.3) (layer "F.Cu") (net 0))
 (segment (start 129.21415 54.0002) (end 147.0202 71.80625) (width 0.3) (layer "F.Cu") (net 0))
 (segment (start 148.3806 72.17175) (end 148.3806 65.8856) (width 0.3) (layer "F.Cu") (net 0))
 (segment (start 145.7352 99.7352) (end 144.4652 99.7352) (width 0.3) (layer "F.Cu") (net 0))
 (segment (start 152.7352 63.1352) (end 152.7352 61.6202) (width 0.3) (layer "F.Cu") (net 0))
 (segment (start 126.8272 104.8764) (end 131.704 104.8764) (width 0.3) (layer "F.Cu") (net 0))
 (segment (start 150.1577 63.1602) (end 150.1952 63.1227) (width 0.3) (layer "F.Cu") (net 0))
 (segment (start 141.991 104.9018) (end 142.0776 104.8152) (width 0.3) (layer "F.Cu") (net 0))
 (segment (start 144.4802 94.6402) (end 144.4652 94.6552) (width 0.3) (layer "F.Cu") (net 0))
 (segment (start 136.8602 119.3102) (end 136.8452 119.2952) (width 0.8) (layer "F.Cu") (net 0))
 (segment (start 127.8272 89.6364) (end 131.7388 85.7248) (width 0.2) (layer "F.Cu") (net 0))
 (segment (start 150.2077 65.1852) (end 150.1952 65.1977) (width 0.3) (layer "F.Cu") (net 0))
 (segment (start 156.336869 138.8362) (end 161.2882 133.884869) (width 0.8) (layer "F.Cu") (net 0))
 (segment (start 133.1552 103.4252) (end 140.1402 103.4252) (width 0.3) (layer "F.Cu") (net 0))
 (segment (start 130.942 132.8164) (end 135.7172 128.0412) (width 0.8) (layer "F.Cu") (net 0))
 (segment (start 147.6552 63.1602) (end 150.1577 63.1602) (width 0.3) (layer "F.Cu") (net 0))
 (segment (start 126.8272 84.5564) (end 142.0164 84.5564) (width 0.8) (layer "F.Cu") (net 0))
 (segment (start 155.4022 50.0632) (end 150.8302 50.0632) (width 0.8) (layer "F.Cu") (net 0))
 (segment (start 146.3598 89.4332) (end 146.3598 72.2882) (width 0.3) (layer "F.Cu") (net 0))
 (segment (start 149.0522 91.0842) (end 149.0522 112.9282) (width 0.8) (layer "F.Cu") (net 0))
 (segment (start 139.1462 50.0632) (end 150.8302 50.0632) (width 0.8) (layer "F.Cu") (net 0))
 (segment (start 152.7352 61.6202) (end 156.4182 61.6202) (width 0.3) (layer "F.Cu") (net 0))
 (segment (start 131.7388 85.7248) (end 132.1358 85.7248) (width 0.2) (layer "F.Cu") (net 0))
 (via (at 147.6806 71.8818) (size 0.6) (drill 0.3) (layers "F.Cu" "B.Cu") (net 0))
 (via (at 132.1358 85.7248) (size 0.6) (drill 0.3) (layers "F.Cu" "B.Cu") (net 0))
 (via (at 142.0164 84.5564) (size 0.6) (drill 0.3) (layers "F.Cu" "B.Cu") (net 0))
 (via (at 130.5102 86.0804) (size 0.6) (drill 0.3) (layers "F.Cu" "B.Cu") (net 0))
 (via (at 131.0182 84.5564) (size 0.5) (drill 0.3) (layers "F.Cu" "B.Cu") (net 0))
 (via (at 140.3908 66.3192) (size 0.6) (drill 0.3) (layers "F.Cu" "B.Cu") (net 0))
 (via (at 130.942 132.8164) (size 0.5) (drill 0.3) (layers "F.Cu" "B.Cu") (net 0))
 (via (at 150.8302 94.640192) (size 0.6) (drill 0.3) (layers "F.Cu" "B.Cu") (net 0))
 (via (at 157.669542 89.795542) (size 0.5) (drill 0.3) (layers "F.Cu" "B.Cu") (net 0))
 (segment (start 136.103854 108.6102) (end 143.2102 108.6102) (width 0.3) (layer "B.Cu") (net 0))
 (segment (start 142.0164 84.5564) (end 142.0926 84.4802) (width 0.8) (layer "B.Cu") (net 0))
 (segment (start 134.3202 92.7352) (end 137.6252 92.7352) (width 0.3) (layer "B.Cu") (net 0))
 (segment (start 126.7002 56.5402) (end 130.6118 56.5402) (width 0.3) (layer "B.Cu") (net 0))
 (segment (start 133.0502 94.0052) (end 134.3202 92.7352) (width 0.3) (layer "B.Cu") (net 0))
 (segment (start 152.2526 92.4558) (end 152.2526 115.8238) (width 0.3) (layer "B.Cu") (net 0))
 (segment (start 152.7526 91.1778) (end 148.7362 87.1614) (width 0.3) (layer "B.Cu") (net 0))
 (segment (start 133.6852 102.2602) (end 133.6852 97.8152) (width 0.3) (layer "B.Cu") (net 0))
 (segment (start 126.8272 109.9564) (end 126.9 110.0292) (width 0.3) (layer "B.Cu") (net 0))
 (segment (start 147.219869 135.1532) (end 148.7882 133.584869) (width 0.3) (layer "B.Cu") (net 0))
 (segment (start 153.8274 116.4842) (end 153.8528 116.5096) (width 0.2) (layer "B.Cu") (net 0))
 (segment (start 126.8272 104.8764) (end 131.069 104.8764) (width 0.3) (layer "B.Cu") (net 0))
 (segment (start 131.007 86.5772) (end 130.5102 86.0804) (width 0.3) (layer "B.Cu") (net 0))
 (segment (start 143.2482 125.535307) (end 152.7526 116.030907) (width 0.3) (layer "B.Cu") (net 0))
 (segment (start 153.3702 84.4802) (end 157.669542 88.779542) (width 0.8) (layer "B.Cu") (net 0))
 (segment (start 152.2526 115.8238) (end 141.8132 126.2632) (width 0.3) (layer "B.Cu") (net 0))
 (segment (start 134.757654 109.9564) (end 136.103854 108.6102) (width 0.3) (layer "B.Cu") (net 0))
 (segment (start 126.8272 102.3364) (end 131.239 102.3364) (width 0.3) (layer "B.Cu") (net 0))
 (segment (start 149.484 85.8772) (end 132.2882 85.8772) (width 0.3) (layer "B.Cu") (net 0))
 (segment (start 126.8272 132.8164) (end 130.942 132.8164) (width 0.8) (layer "B.Cu") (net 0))
 (segment (start 153.8782 90.2714) (end 149.484 85.8772) (width 0.3) (layer "B.Cu") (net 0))
 (segment (start 143.2482 133.584869) (end 143.2482 125.535307) (width 0.3) (layer "B.Cu") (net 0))
 (segment (start 126.8272 107.4164) (end 134.757654 107.4164) (width 0.3) (layer "B.Cu") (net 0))
 (segment (start 146.0182 123.5822) (end 153.3702 116.2302) (width 0.3) (layer "B.Cu") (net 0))
 (segment (start 131.0182 69.2402) (end 145.039 69.2402) (width 0.3) (layer "B.Cu") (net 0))
 (segment (start 126.8922 87.1614) (end 126.8272 87.0964) (width 0.3) (layer "B.Cu") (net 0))
 (segment (start 149.2188 86.5772) (end 131.007 86.5772) (width 0.3) (layer "B.Cu") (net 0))
 (segment (start 134.757654 107.4164) (end 136.103854 106.0702) (width 0.3) (layer "B.Cu") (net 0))
 (segment (start 145.039 69.2402) (end 147.6806 71.8818) (width 0.3) (layer "B.Cu") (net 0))
 (segment (start 150.815192 94.6552) (end 150.8302 94.640192) (width 0.8) (layer "B.Cu") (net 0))
 (segment (start 153.3194 116.1794) (end 153.3194 90.6778) (width 0.3) (layer "B.Cu") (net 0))
 (segment (start 151.5582 118.8042) (end 153.8528 116.5096) (width 0.3) (layer "B.Cu") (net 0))
 (segment (start 126.8272 107.4164) (end 126.9 107.4892) (width 0.3) (layer "B.Cu") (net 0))
 (segment (start 138.7502 99.7352) (end 136.8452 99.7352) (width 0.3) (layer "B.Cu") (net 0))
 (segment (start 126.8272 89.6364) (end 149.4332 89.6364) (width 0.3) (layer "B.Cu") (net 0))
 (segment (start 142.0926 84.4802) (end 153.3702 84.4802) (width 0.8) (layer "B.Cu") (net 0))
 (segment (start 133.6852 97.8152) (end 136.8452 94.6552) (width 0.3) (layer "B.Cu") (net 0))
 (segment (start 136.8452 104.8152) (end 136.8452 102.2752) (width 0.3) (layer "B.Cu") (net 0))
 (segment (start 131.0182 69.2402) (end 126.7002 69.2402) (width 0.3) (layer "B.Cu") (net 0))
 (segment (start 144.4652 94.6552) (end 150.815192 94.6552) (width 0.8) (layer "B.Cu") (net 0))
 (segment (start 153.8782 116.4334) (end 153.8782 90.2714) (width 0.3) (layer "B.Cu") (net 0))
 (segment (start 131.069 104.8764) (end 133.6852 102.2602) (width 0.3) (layer "B.Cu") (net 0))
 (segment (start 139.4002 99.0852) (end 138.7502 99.7352) (width 0.3) (layer "B.Cu") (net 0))
 (segment (start 149.4332 89.6364) (end 152.2526 92.4558) (width 0.3) (layer "B.Cu") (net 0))
 (segment (start 132.2882 85.8772) (end 132.1358 85.7248) (width 0.3) (layer "B.Cu") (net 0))
 (segment (start 140.6702 106.0702) (end 144.4652 102.2752) (width 0.3) (layer "B.Cu") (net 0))
 (segment (start 153.8274 116.4842) (end 153.8782 116.4334) (width 0.3) (layer "B.Cu") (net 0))
 (segment (start 139.4002 94.5102) (end 139.4002 99.0852) (width 0.3) (layer "B.Cu") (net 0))
 (segment (start 130.6118 56.5402) (end 140.3908 66.3192) (width 0.3) (layer "B.Cu") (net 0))
 (segment (start 141.8132 135.1532) (end 147.219869 135.1532) (width 0.3) (layer "B.Cu") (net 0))
 (segment (start 137.6252 92.7352) (end 139.4002 94.5102) (width 0.3) (layer "B.Cu") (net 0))
 (segment (start 131.0182 84.5564) (end 126.8272 84.5564) (width 0.8) (layer "B.Cu") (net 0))
 (segment (start 143.2102 108.6102) (end 144.4652 107.3552) (width 0.3) (layer "B.Cu") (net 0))
 (segment (start 133.0502 100.5252) (end 133.0502 94.0052) (width 0.3) (layer "B.Cu") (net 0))
 (segment (start 157.669542 88.779542) (end 157.669542 89.795542) (width 0.8) (layer "B.Cu") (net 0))
 (segment (start 146.0182 133.584869) (end 146.0182 123.5822) (width 0.3) (layer "B.Cu") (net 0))
 (segment (start 153.3194 116.1794) (end 153.3702 116.2302) (width 0.2) (layer "B.Cu") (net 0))
 (segment (start 141.8132 126.2632) (end 141.8132 135.1532) (width 0.3) (layer "B.Cu") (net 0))
 (segment (start 126.8272 109.9564) (end 134.757654 109.9564) (width 0.3) (layer "B.Cu") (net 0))
 (segment (start 131.239 102.3364) (end 133.0502 100.5252) (width 0.3) (layer "B.Cu") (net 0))
 (segment (start 153.3194 90.6778) (end 149.2188 86.5772) (width 0.3) (layer "B.Cu") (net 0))
 (segment (start 148.7362 87.1614) (end 126.8922 87.1614) (width 0.3) (layer "B.Cu") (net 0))
 (segment (start 152.7526 116.030907) (end 152.7526 91.1778) (width 0.3) (layer "B.Cu") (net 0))
 (segment (start 151.5582 133.584869) (end 151.5582 118.8042) (width 0.3) (layer "B.Cu") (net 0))
 (segment (start 136.103854 106.0702) (end 140.6702 106.0702) (width 0.3) (layer "B.Cu") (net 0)))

